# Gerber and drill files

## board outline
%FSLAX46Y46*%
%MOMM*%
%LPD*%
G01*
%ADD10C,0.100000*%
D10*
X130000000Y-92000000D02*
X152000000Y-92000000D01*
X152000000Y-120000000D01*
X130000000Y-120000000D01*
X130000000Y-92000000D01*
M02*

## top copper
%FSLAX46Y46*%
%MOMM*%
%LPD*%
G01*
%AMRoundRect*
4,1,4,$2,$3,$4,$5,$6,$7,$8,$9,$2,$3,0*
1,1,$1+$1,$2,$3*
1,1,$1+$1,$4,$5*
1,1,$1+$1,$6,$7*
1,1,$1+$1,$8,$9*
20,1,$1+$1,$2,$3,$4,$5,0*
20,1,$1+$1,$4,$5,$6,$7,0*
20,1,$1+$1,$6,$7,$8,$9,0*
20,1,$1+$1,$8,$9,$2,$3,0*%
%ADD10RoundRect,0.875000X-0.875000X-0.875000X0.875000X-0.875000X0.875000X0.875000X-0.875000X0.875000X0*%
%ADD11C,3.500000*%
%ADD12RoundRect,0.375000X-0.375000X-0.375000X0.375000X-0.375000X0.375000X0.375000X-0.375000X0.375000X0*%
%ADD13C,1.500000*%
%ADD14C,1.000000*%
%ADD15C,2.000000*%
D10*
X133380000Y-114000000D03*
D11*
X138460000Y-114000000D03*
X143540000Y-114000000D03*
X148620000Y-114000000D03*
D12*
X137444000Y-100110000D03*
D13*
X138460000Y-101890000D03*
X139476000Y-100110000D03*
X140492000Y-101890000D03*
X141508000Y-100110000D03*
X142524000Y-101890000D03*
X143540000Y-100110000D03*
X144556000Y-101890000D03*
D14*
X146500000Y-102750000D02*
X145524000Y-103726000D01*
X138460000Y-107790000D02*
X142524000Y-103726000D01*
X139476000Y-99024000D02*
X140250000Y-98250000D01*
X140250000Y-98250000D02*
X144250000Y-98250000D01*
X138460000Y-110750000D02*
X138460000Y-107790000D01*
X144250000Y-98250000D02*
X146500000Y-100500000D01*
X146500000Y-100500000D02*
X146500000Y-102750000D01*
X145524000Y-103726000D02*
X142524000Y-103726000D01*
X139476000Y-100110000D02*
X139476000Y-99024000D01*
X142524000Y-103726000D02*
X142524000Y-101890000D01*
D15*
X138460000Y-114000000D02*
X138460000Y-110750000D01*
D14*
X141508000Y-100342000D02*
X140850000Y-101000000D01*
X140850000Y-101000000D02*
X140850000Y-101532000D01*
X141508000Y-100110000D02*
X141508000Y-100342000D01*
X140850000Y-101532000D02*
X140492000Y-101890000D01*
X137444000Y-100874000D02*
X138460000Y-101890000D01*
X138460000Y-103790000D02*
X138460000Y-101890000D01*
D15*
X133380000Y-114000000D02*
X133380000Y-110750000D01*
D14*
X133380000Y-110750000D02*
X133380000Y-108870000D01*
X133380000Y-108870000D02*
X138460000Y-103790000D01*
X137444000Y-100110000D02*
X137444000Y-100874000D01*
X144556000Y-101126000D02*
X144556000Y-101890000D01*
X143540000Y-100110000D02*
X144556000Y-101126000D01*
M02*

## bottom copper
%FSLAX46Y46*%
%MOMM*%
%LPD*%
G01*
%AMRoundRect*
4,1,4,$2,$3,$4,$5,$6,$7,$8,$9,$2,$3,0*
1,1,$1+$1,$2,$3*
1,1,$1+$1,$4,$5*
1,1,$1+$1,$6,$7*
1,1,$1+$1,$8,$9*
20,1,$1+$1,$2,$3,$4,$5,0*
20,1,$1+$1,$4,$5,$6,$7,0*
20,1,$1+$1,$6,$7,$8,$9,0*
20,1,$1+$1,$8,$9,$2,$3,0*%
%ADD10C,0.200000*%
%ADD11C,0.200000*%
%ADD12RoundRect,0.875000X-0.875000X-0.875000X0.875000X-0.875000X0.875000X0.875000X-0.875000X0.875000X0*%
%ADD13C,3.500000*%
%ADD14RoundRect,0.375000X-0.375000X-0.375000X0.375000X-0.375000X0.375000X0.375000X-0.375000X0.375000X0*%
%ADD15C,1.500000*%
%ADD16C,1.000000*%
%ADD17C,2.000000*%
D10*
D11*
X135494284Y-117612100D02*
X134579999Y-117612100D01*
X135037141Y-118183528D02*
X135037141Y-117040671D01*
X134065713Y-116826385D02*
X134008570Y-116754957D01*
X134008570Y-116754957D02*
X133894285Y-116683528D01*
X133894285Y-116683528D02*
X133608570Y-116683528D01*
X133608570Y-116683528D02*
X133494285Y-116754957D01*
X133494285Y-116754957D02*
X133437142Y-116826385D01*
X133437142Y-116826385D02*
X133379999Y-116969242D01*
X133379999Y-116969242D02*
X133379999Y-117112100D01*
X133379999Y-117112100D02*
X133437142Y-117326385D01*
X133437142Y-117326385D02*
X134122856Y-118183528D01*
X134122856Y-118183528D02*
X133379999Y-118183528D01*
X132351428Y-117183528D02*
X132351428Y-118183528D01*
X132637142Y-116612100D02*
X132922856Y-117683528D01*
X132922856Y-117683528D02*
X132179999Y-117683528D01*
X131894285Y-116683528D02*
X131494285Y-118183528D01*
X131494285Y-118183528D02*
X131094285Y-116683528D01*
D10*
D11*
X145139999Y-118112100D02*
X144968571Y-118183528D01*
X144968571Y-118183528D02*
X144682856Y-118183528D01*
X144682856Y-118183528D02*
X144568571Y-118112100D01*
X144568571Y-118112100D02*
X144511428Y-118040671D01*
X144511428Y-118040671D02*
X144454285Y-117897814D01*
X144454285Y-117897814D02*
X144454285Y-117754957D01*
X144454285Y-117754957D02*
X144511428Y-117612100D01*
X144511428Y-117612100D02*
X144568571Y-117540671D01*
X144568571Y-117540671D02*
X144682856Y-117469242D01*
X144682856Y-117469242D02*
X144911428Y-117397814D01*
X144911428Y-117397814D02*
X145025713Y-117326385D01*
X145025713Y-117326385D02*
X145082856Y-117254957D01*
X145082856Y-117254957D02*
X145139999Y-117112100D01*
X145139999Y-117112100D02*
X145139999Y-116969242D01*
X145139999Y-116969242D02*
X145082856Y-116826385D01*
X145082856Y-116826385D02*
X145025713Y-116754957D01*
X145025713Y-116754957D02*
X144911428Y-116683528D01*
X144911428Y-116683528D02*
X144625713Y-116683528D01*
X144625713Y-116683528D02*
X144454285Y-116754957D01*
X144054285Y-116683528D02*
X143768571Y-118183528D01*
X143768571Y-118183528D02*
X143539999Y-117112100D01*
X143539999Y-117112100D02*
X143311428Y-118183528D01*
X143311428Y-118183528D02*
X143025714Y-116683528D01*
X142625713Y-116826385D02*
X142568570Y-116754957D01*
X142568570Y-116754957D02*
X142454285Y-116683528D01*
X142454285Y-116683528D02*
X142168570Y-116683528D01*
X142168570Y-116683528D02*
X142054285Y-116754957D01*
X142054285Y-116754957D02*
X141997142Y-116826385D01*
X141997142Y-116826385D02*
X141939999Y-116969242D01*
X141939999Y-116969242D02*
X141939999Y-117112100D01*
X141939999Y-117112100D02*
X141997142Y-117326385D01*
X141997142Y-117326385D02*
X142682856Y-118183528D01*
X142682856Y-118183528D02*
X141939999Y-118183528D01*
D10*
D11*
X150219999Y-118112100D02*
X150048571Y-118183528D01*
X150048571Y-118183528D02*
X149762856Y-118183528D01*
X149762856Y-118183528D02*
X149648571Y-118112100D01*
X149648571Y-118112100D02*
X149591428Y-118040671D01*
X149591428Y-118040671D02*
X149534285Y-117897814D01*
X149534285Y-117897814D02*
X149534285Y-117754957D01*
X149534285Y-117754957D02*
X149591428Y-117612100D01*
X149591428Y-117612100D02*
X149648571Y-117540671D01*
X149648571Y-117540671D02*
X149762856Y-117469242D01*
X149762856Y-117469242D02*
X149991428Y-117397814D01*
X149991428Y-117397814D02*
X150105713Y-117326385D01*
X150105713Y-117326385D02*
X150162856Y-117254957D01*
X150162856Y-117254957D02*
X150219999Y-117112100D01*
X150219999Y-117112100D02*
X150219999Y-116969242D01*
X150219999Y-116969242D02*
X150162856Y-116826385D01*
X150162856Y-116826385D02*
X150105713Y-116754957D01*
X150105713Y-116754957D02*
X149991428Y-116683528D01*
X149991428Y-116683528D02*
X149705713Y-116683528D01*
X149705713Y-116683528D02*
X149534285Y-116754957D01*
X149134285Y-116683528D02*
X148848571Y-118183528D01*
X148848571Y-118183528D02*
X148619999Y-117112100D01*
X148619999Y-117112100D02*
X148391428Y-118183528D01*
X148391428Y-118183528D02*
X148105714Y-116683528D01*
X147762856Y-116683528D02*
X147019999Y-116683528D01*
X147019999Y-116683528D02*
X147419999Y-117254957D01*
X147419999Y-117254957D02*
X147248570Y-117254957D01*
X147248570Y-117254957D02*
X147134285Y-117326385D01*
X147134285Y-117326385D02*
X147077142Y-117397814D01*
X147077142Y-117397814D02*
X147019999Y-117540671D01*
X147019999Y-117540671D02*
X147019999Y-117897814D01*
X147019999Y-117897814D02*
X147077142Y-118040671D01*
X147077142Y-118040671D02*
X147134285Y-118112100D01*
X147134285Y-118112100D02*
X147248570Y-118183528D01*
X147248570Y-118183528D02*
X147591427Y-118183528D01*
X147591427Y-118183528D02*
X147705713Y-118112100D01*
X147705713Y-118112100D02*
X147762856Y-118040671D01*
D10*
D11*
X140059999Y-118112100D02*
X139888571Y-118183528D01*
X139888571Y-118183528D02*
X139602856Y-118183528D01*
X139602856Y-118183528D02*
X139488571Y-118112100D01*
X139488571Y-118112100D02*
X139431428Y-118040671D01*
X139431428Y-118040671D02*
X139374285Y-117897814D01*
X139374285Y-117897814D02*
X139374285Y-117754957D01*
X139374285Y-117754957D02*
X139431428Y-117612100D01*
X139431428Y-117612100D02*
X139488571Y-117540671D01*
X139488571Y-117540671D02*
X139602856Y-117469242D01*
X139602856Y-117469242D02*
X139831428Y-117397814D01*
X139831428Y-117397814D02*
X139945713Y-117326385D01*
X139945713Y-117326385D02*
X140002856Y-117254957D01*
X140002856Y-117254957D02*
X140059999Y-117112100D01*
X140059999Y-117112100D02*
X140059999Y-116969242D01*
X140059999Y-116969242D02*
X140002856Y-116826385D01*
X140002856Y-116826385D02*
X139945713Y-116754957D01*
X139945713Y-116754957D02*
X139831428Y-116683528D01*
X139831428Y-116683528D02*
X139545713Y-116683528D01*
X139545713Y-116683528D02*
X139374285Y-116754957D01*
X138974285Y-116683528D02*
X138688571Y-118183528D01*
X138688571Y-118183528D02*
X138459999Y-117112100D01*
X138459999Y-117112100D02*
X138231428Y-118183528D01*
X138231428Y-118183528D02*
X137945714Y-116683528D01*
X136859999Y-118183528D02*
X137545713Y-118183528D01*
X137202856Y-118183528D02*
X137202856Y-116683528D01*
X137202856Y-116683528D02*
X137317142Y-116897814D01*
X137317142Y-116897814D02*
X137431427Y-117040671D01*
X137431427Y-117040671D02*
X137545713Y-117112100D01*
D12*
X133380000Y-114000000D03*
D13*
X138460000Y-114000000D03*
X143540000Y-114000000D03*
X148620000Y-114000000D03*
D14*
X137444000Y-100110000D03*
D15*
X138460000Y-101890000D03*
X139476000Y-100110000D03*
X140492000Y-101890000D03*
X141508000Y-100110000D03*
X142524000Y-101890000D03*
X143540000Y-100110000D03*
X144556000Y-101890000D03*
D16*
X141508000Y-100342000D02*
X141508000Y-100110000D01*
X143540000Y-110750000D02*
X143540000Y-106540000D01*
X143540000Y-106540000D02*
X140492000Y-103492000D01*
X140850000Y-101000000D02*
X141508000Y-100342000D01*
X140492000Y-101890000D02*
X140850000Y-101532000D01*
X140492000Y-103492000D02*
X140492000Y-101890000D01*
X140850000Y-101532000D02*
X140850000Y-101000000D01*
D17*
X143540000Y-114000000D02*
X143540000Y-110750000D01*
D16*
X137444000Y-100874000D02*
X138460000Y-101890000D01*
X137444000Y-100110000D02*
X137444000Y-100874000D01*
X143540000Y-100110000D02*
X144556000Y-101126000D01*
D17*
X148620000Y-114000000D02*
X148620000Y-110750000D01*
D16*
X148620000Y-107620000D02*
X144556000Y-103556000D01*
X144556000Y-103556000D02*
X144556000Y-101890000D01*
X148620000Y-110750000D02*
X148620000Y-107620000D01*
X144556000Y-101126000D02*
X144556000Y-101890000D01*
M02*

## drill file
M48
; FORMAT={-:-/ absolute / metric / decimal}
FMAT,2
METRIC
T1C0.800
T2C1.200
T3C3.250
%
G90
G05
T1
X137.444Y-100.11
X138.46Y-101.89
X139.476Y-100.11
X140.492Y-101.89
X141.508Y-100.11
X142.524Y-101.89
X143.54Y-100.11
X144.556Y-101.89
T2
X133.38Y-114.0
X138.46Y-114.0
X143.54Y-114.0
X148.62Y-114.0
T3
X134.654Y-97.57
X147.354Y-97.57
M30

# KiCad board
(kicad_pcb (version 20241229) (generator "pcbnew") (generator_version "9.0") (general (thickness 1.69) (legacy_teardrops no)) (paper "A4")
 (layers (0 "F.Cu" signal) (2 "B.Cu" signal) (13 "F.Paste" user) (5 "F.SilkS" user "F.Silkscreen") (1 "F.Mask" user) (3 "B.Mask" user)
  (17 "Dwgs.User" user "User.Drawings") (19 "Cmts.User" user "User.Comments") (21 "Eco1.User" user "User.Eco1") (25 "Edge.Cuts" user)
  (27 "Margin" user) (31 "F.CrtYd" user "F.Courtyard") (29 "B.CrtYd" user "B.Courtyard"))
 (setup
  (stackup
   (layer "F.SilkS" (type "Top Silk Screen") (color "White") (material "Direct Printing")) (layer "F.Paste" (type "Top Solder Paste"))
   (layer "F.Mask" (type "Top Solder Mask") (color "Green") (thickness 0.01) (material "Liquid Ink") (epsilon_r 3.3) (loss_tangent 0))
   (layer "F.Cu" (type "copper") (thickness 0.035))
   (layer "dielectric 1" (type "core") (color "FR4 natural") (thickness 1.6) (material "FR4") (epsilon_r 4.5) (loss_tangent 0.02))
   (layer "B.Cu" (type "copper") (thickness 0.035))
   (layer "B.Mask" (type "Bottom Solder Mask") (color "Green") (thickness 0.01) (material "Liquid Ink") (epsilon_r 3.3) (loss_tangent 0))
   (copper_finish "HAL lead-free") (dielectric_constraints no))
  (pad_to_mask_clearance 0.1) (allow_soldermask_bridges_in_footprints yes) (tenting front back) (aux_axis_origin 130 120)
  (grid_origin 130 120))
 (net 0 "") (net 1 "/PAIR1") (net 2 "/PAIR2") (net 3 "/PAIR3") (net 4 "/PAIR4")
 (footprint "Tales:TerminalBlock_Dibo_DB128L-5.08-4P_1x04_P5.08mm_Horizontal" (layer "F.Cu") (at 141 114)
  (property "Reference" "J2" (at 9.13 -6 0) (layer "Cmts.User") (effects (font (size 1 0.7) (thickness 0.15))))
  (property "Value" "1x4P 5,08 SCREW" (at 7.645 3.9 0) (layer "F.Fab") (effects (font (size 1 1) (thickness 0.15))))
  (pad "1" thru_hole roundrect (at -7.62 0) (size 3.5 3.5) (drill 1.2) (layers "*.Cu" "*.Mask") (remove_unused_layers no)
   (roundrect_rratio 0.25) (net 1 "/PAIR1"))
  (pad "2" thru_hole circle (at -2.54 0) (size 3.5 3.5) (drill 1.2) (layers "*.Cu" "*.Mask") (remove_unused_layers no) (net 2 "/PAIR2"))
  (pad "3" thru_hole circle (at 2.54 0) (size 3.5 3.5) (drill 1.2) (layers "*.Cu" "*.Mask") (remove_unused_layers no) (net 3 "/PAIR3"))
  (pad "4" thru_hole circle (at 7.62 0) (size 3.5 3.5) (drill 1.2) (layers "*.Cu" "*.Mask") (remove_unused_layers no) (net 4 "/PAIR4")))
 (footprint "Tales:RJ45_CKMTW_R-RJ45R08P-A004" (layer "F.Cu") (at 141 101 180)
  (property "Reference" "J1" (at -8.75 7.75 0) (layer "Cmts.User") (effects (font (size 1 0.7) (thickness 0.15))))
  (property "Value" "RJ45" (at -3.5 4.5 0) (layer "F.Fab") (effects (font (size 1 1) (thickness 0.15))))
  (pad "" np_thru_hole circle (at -6.354 3.43) (size 3.25 3.25) (drill 3.25) (layers "*.Cu" "*.Mask"))
  (pad "" np_thru_hole circle (at 6.346 3.43) (size 3.25 3.25) (drill 3.25) (layers "*.Cu" "*.Mask"))
  (pad "1" thru_hole roundrect (at 3.556 0.89) (size 1.5 1.5) (drill 0.8) (layers "*.Cu" "*.Mask") (remove_unused_layers no)
   (roundrect_rratio 0.25) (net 1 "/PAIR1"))
  (pad "2" thru_hole circle (at 2.54 -0.89) (size 1.5 1.5) (drill 0.8) (layers "*.Cu" "*.Mask") (remove_unused_layers no) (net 1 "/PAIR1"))
  (pad "3" thru_hole circle (at 1.524 0.89) (size 1.5 1.5) (drill 0.8) (layers "*.Cu" "*.Mask") (remove_unused_layers no) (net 2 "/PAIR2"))
  (pad "4" thru_hole circle (at 0.508 -0.89) (size 1.5 1.5) (drill 0.8) (layers "*.Cu" "*.Mask") (remove_unused_layers no) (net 3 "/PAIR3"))
  (pad "5" thru_hole circle (at -0.508 0.89) (size 1.5 1.5) (drill 0.8) (layers "*.Cu" "*.Mask") (remove_unused_layers no) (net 3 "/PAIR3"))
  (pad "6" thru_hole circle (at -1.524 -0.89) (size 1.5 1.5) (drill 0.8) (layers "*.Cu" "*.Mask") (remove_unused_layers no) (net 2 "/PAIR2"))
  (pad "7" thru_hole circle (at -2.54 0.89) (size 1.5 1.5) (drill 0.8) (layers "*.Cu" "*.Mask") (remove_unused_layers no) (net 4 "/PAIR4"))
  (pad "8" thru_hole circle (at -3.556 -0.89) (size 1.5 1.5) (drill 0.8) (layers "*.Cu" "*.Mask") (remove_unused_layers no) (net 4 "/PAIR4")))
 (gr_rect (start 130 92) (end 152 120) (stroke (width 0.1) (type default)) (fill no) (layer "Edge.Cuts"))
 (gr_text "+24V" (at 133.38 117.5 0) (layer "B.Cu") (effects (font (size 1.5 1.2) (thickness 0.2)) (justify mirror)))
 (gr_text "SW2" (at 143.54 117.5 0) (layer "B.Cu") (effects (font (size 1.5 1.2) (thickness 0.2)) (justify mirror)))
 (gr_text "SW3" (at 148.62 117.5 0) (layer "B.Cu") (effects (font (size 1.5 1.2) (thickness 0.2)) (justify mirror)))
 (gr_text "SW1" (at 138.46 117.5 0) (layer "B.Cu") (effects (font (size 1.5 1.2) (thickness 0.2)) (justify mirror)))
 (segment (start 146.5 102.75) (end 145.524 103.726) (width 1) (layer "F.Cu") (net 2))
 (segment (start 138.46 107.79) (end 142.524 103.726) (width 1) (layer "F.Cu") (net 2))
 (segment (start 139.476 99.024) (end 140.25 98.25) (width 1) (layer "F.Cu") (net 2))
 (segment (start 140.25 98.25) (end 144.25 98.25) (width 1) (layer "F.Cu") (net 2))
 (segment (start 138.46 110.75) (end 138.46 107.79) (width 1) (layer "F.Cu") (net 2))
 (segment (start 144.25 98.25) (end 146.5 100.5) (width 1) (layer "F.Cu") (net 2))
 (segment (start 146.5 100.5) (end 146.5 102.75) (width 1) (layer "F.Cu") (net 2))
 (segment (start 145.524 103.726) (end 142.524 103.726) (width 1) (layer "F.Cu") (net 2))
 (segment (start 139.476 100.11) (end 139.476 99.024) (width 1) (layer "F.Cu") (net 2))
 (segment (start 142.524 103.726) (end 142.524 101.89) (width 1) (layer "F.Cu") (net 2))
 (segment (start 138.46 114) (end 138.46 110.75) (width 2) (layer "F.Cu") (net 2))
 (segment (start 141.508 100.342) (end 140.85 101) (width 1) (layer "F.Cu") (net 3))
 (segment (start 140.85 101) (end 140.85 101.532) (width 1) (layer "F.Cu") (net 3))
 (segment (start 141.508 100.11) (end 141.508 100.342) (width 1) (layer "F.Cu") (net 3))
 (segment (start 140.85 101.532) (end 140.492 101.89) (width 1) (layer "F.Cu") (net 3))
 (segment (start 141.508 100.342) (end 141.508 100.11) (width 1) (layer "B.Cu") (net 3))
 (segment (start 143.54 110.75) (end 143.54 106.54) (width 1) (layer "B.Cu") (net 3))
 (segment (start 143.54 106.54) (end 140.492 103.492) (width 1) (layer "B.Cu") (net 3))
 (segment (start 140.85 101) (end 141.508 100.342) (width 1) (layer "B.Cu") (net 3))
 (segment (start 140.492 101.89) (end 140.85 101.532) (width 1) (layer "B.Cu") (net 3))
 (segment (start 140.492 103.492) (end 140.492 101.89) (width 1) (layer "B.Cu") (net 3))
 (segment (start 140.85 101.532) (end 140.85 101) (width 1) (layer "B.Cu") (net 3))
 (segment (start 143.54 114) (end 143.54 110.75) (width 2) (layer "B.Cu") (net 3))
 (segment (start 137.444 100.874) (end 138.46 101.89) (width 1) (layer "F.Cu") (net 1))
 (segment (start 138.46 103.79) (end 138.46 101.89) (width 1) (layer "F.Cu") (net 1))
 (segment (start 133.38 114) (end 133.38 110.75) (width 2) (layer "F.Cu") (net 1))
 (segment (start 133.38 110.75) (end 133.38 108.87) (width 1) (layer "F.Cu") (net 1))
 (segment (start 133.38 108.87) (end 138.46 103.79) (width 1) (layer "F.Cu") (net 1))
 (segment (start 137.444 100.11) (end 137.444 100.874) (width 1) (layer "F.Cu") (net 1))
 (segment (start 137.444 100.874) (end 138.46 101.89) (width 1) (layer "B.Cu") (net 1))
 (segment (start 137.444 100.11) (end 137.444 100.874) (width 1) (layer "B.Cu") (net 1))
 (segment (start 144.556 101.126) (end 144.556 101.89) (width 1) (layer "F.Cu") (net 4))
 (segment (start 143.54 100.11) (end 144.556 101.126) (width 1) (layer "F.Cu") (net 4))
 (segment (start 143.54 100.11) (end 144.556 101.126) (width 1) (layer "B.Cu") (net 4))
 (segment (start 148.62 114) (end 148.62 110.75) (width 2) (layer "B.Cu") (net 4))
 (segment (start 148.62 107.62) (end 144.556 103.556) (width 1) (layer "B.Cu") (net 4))
 (segment (start 144.556 103.556) (end 144.556 101.89) (width 1) (layer "B.Cu") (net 4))
 (segment (start 148.62 110.75) (end 148.62 107.62) (width 1) (layer "B.Cu") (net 4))
 (segment (start 144.556 101.126) (end 144.556 101.89) (width 1) (layer "B.Cu") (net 4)))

